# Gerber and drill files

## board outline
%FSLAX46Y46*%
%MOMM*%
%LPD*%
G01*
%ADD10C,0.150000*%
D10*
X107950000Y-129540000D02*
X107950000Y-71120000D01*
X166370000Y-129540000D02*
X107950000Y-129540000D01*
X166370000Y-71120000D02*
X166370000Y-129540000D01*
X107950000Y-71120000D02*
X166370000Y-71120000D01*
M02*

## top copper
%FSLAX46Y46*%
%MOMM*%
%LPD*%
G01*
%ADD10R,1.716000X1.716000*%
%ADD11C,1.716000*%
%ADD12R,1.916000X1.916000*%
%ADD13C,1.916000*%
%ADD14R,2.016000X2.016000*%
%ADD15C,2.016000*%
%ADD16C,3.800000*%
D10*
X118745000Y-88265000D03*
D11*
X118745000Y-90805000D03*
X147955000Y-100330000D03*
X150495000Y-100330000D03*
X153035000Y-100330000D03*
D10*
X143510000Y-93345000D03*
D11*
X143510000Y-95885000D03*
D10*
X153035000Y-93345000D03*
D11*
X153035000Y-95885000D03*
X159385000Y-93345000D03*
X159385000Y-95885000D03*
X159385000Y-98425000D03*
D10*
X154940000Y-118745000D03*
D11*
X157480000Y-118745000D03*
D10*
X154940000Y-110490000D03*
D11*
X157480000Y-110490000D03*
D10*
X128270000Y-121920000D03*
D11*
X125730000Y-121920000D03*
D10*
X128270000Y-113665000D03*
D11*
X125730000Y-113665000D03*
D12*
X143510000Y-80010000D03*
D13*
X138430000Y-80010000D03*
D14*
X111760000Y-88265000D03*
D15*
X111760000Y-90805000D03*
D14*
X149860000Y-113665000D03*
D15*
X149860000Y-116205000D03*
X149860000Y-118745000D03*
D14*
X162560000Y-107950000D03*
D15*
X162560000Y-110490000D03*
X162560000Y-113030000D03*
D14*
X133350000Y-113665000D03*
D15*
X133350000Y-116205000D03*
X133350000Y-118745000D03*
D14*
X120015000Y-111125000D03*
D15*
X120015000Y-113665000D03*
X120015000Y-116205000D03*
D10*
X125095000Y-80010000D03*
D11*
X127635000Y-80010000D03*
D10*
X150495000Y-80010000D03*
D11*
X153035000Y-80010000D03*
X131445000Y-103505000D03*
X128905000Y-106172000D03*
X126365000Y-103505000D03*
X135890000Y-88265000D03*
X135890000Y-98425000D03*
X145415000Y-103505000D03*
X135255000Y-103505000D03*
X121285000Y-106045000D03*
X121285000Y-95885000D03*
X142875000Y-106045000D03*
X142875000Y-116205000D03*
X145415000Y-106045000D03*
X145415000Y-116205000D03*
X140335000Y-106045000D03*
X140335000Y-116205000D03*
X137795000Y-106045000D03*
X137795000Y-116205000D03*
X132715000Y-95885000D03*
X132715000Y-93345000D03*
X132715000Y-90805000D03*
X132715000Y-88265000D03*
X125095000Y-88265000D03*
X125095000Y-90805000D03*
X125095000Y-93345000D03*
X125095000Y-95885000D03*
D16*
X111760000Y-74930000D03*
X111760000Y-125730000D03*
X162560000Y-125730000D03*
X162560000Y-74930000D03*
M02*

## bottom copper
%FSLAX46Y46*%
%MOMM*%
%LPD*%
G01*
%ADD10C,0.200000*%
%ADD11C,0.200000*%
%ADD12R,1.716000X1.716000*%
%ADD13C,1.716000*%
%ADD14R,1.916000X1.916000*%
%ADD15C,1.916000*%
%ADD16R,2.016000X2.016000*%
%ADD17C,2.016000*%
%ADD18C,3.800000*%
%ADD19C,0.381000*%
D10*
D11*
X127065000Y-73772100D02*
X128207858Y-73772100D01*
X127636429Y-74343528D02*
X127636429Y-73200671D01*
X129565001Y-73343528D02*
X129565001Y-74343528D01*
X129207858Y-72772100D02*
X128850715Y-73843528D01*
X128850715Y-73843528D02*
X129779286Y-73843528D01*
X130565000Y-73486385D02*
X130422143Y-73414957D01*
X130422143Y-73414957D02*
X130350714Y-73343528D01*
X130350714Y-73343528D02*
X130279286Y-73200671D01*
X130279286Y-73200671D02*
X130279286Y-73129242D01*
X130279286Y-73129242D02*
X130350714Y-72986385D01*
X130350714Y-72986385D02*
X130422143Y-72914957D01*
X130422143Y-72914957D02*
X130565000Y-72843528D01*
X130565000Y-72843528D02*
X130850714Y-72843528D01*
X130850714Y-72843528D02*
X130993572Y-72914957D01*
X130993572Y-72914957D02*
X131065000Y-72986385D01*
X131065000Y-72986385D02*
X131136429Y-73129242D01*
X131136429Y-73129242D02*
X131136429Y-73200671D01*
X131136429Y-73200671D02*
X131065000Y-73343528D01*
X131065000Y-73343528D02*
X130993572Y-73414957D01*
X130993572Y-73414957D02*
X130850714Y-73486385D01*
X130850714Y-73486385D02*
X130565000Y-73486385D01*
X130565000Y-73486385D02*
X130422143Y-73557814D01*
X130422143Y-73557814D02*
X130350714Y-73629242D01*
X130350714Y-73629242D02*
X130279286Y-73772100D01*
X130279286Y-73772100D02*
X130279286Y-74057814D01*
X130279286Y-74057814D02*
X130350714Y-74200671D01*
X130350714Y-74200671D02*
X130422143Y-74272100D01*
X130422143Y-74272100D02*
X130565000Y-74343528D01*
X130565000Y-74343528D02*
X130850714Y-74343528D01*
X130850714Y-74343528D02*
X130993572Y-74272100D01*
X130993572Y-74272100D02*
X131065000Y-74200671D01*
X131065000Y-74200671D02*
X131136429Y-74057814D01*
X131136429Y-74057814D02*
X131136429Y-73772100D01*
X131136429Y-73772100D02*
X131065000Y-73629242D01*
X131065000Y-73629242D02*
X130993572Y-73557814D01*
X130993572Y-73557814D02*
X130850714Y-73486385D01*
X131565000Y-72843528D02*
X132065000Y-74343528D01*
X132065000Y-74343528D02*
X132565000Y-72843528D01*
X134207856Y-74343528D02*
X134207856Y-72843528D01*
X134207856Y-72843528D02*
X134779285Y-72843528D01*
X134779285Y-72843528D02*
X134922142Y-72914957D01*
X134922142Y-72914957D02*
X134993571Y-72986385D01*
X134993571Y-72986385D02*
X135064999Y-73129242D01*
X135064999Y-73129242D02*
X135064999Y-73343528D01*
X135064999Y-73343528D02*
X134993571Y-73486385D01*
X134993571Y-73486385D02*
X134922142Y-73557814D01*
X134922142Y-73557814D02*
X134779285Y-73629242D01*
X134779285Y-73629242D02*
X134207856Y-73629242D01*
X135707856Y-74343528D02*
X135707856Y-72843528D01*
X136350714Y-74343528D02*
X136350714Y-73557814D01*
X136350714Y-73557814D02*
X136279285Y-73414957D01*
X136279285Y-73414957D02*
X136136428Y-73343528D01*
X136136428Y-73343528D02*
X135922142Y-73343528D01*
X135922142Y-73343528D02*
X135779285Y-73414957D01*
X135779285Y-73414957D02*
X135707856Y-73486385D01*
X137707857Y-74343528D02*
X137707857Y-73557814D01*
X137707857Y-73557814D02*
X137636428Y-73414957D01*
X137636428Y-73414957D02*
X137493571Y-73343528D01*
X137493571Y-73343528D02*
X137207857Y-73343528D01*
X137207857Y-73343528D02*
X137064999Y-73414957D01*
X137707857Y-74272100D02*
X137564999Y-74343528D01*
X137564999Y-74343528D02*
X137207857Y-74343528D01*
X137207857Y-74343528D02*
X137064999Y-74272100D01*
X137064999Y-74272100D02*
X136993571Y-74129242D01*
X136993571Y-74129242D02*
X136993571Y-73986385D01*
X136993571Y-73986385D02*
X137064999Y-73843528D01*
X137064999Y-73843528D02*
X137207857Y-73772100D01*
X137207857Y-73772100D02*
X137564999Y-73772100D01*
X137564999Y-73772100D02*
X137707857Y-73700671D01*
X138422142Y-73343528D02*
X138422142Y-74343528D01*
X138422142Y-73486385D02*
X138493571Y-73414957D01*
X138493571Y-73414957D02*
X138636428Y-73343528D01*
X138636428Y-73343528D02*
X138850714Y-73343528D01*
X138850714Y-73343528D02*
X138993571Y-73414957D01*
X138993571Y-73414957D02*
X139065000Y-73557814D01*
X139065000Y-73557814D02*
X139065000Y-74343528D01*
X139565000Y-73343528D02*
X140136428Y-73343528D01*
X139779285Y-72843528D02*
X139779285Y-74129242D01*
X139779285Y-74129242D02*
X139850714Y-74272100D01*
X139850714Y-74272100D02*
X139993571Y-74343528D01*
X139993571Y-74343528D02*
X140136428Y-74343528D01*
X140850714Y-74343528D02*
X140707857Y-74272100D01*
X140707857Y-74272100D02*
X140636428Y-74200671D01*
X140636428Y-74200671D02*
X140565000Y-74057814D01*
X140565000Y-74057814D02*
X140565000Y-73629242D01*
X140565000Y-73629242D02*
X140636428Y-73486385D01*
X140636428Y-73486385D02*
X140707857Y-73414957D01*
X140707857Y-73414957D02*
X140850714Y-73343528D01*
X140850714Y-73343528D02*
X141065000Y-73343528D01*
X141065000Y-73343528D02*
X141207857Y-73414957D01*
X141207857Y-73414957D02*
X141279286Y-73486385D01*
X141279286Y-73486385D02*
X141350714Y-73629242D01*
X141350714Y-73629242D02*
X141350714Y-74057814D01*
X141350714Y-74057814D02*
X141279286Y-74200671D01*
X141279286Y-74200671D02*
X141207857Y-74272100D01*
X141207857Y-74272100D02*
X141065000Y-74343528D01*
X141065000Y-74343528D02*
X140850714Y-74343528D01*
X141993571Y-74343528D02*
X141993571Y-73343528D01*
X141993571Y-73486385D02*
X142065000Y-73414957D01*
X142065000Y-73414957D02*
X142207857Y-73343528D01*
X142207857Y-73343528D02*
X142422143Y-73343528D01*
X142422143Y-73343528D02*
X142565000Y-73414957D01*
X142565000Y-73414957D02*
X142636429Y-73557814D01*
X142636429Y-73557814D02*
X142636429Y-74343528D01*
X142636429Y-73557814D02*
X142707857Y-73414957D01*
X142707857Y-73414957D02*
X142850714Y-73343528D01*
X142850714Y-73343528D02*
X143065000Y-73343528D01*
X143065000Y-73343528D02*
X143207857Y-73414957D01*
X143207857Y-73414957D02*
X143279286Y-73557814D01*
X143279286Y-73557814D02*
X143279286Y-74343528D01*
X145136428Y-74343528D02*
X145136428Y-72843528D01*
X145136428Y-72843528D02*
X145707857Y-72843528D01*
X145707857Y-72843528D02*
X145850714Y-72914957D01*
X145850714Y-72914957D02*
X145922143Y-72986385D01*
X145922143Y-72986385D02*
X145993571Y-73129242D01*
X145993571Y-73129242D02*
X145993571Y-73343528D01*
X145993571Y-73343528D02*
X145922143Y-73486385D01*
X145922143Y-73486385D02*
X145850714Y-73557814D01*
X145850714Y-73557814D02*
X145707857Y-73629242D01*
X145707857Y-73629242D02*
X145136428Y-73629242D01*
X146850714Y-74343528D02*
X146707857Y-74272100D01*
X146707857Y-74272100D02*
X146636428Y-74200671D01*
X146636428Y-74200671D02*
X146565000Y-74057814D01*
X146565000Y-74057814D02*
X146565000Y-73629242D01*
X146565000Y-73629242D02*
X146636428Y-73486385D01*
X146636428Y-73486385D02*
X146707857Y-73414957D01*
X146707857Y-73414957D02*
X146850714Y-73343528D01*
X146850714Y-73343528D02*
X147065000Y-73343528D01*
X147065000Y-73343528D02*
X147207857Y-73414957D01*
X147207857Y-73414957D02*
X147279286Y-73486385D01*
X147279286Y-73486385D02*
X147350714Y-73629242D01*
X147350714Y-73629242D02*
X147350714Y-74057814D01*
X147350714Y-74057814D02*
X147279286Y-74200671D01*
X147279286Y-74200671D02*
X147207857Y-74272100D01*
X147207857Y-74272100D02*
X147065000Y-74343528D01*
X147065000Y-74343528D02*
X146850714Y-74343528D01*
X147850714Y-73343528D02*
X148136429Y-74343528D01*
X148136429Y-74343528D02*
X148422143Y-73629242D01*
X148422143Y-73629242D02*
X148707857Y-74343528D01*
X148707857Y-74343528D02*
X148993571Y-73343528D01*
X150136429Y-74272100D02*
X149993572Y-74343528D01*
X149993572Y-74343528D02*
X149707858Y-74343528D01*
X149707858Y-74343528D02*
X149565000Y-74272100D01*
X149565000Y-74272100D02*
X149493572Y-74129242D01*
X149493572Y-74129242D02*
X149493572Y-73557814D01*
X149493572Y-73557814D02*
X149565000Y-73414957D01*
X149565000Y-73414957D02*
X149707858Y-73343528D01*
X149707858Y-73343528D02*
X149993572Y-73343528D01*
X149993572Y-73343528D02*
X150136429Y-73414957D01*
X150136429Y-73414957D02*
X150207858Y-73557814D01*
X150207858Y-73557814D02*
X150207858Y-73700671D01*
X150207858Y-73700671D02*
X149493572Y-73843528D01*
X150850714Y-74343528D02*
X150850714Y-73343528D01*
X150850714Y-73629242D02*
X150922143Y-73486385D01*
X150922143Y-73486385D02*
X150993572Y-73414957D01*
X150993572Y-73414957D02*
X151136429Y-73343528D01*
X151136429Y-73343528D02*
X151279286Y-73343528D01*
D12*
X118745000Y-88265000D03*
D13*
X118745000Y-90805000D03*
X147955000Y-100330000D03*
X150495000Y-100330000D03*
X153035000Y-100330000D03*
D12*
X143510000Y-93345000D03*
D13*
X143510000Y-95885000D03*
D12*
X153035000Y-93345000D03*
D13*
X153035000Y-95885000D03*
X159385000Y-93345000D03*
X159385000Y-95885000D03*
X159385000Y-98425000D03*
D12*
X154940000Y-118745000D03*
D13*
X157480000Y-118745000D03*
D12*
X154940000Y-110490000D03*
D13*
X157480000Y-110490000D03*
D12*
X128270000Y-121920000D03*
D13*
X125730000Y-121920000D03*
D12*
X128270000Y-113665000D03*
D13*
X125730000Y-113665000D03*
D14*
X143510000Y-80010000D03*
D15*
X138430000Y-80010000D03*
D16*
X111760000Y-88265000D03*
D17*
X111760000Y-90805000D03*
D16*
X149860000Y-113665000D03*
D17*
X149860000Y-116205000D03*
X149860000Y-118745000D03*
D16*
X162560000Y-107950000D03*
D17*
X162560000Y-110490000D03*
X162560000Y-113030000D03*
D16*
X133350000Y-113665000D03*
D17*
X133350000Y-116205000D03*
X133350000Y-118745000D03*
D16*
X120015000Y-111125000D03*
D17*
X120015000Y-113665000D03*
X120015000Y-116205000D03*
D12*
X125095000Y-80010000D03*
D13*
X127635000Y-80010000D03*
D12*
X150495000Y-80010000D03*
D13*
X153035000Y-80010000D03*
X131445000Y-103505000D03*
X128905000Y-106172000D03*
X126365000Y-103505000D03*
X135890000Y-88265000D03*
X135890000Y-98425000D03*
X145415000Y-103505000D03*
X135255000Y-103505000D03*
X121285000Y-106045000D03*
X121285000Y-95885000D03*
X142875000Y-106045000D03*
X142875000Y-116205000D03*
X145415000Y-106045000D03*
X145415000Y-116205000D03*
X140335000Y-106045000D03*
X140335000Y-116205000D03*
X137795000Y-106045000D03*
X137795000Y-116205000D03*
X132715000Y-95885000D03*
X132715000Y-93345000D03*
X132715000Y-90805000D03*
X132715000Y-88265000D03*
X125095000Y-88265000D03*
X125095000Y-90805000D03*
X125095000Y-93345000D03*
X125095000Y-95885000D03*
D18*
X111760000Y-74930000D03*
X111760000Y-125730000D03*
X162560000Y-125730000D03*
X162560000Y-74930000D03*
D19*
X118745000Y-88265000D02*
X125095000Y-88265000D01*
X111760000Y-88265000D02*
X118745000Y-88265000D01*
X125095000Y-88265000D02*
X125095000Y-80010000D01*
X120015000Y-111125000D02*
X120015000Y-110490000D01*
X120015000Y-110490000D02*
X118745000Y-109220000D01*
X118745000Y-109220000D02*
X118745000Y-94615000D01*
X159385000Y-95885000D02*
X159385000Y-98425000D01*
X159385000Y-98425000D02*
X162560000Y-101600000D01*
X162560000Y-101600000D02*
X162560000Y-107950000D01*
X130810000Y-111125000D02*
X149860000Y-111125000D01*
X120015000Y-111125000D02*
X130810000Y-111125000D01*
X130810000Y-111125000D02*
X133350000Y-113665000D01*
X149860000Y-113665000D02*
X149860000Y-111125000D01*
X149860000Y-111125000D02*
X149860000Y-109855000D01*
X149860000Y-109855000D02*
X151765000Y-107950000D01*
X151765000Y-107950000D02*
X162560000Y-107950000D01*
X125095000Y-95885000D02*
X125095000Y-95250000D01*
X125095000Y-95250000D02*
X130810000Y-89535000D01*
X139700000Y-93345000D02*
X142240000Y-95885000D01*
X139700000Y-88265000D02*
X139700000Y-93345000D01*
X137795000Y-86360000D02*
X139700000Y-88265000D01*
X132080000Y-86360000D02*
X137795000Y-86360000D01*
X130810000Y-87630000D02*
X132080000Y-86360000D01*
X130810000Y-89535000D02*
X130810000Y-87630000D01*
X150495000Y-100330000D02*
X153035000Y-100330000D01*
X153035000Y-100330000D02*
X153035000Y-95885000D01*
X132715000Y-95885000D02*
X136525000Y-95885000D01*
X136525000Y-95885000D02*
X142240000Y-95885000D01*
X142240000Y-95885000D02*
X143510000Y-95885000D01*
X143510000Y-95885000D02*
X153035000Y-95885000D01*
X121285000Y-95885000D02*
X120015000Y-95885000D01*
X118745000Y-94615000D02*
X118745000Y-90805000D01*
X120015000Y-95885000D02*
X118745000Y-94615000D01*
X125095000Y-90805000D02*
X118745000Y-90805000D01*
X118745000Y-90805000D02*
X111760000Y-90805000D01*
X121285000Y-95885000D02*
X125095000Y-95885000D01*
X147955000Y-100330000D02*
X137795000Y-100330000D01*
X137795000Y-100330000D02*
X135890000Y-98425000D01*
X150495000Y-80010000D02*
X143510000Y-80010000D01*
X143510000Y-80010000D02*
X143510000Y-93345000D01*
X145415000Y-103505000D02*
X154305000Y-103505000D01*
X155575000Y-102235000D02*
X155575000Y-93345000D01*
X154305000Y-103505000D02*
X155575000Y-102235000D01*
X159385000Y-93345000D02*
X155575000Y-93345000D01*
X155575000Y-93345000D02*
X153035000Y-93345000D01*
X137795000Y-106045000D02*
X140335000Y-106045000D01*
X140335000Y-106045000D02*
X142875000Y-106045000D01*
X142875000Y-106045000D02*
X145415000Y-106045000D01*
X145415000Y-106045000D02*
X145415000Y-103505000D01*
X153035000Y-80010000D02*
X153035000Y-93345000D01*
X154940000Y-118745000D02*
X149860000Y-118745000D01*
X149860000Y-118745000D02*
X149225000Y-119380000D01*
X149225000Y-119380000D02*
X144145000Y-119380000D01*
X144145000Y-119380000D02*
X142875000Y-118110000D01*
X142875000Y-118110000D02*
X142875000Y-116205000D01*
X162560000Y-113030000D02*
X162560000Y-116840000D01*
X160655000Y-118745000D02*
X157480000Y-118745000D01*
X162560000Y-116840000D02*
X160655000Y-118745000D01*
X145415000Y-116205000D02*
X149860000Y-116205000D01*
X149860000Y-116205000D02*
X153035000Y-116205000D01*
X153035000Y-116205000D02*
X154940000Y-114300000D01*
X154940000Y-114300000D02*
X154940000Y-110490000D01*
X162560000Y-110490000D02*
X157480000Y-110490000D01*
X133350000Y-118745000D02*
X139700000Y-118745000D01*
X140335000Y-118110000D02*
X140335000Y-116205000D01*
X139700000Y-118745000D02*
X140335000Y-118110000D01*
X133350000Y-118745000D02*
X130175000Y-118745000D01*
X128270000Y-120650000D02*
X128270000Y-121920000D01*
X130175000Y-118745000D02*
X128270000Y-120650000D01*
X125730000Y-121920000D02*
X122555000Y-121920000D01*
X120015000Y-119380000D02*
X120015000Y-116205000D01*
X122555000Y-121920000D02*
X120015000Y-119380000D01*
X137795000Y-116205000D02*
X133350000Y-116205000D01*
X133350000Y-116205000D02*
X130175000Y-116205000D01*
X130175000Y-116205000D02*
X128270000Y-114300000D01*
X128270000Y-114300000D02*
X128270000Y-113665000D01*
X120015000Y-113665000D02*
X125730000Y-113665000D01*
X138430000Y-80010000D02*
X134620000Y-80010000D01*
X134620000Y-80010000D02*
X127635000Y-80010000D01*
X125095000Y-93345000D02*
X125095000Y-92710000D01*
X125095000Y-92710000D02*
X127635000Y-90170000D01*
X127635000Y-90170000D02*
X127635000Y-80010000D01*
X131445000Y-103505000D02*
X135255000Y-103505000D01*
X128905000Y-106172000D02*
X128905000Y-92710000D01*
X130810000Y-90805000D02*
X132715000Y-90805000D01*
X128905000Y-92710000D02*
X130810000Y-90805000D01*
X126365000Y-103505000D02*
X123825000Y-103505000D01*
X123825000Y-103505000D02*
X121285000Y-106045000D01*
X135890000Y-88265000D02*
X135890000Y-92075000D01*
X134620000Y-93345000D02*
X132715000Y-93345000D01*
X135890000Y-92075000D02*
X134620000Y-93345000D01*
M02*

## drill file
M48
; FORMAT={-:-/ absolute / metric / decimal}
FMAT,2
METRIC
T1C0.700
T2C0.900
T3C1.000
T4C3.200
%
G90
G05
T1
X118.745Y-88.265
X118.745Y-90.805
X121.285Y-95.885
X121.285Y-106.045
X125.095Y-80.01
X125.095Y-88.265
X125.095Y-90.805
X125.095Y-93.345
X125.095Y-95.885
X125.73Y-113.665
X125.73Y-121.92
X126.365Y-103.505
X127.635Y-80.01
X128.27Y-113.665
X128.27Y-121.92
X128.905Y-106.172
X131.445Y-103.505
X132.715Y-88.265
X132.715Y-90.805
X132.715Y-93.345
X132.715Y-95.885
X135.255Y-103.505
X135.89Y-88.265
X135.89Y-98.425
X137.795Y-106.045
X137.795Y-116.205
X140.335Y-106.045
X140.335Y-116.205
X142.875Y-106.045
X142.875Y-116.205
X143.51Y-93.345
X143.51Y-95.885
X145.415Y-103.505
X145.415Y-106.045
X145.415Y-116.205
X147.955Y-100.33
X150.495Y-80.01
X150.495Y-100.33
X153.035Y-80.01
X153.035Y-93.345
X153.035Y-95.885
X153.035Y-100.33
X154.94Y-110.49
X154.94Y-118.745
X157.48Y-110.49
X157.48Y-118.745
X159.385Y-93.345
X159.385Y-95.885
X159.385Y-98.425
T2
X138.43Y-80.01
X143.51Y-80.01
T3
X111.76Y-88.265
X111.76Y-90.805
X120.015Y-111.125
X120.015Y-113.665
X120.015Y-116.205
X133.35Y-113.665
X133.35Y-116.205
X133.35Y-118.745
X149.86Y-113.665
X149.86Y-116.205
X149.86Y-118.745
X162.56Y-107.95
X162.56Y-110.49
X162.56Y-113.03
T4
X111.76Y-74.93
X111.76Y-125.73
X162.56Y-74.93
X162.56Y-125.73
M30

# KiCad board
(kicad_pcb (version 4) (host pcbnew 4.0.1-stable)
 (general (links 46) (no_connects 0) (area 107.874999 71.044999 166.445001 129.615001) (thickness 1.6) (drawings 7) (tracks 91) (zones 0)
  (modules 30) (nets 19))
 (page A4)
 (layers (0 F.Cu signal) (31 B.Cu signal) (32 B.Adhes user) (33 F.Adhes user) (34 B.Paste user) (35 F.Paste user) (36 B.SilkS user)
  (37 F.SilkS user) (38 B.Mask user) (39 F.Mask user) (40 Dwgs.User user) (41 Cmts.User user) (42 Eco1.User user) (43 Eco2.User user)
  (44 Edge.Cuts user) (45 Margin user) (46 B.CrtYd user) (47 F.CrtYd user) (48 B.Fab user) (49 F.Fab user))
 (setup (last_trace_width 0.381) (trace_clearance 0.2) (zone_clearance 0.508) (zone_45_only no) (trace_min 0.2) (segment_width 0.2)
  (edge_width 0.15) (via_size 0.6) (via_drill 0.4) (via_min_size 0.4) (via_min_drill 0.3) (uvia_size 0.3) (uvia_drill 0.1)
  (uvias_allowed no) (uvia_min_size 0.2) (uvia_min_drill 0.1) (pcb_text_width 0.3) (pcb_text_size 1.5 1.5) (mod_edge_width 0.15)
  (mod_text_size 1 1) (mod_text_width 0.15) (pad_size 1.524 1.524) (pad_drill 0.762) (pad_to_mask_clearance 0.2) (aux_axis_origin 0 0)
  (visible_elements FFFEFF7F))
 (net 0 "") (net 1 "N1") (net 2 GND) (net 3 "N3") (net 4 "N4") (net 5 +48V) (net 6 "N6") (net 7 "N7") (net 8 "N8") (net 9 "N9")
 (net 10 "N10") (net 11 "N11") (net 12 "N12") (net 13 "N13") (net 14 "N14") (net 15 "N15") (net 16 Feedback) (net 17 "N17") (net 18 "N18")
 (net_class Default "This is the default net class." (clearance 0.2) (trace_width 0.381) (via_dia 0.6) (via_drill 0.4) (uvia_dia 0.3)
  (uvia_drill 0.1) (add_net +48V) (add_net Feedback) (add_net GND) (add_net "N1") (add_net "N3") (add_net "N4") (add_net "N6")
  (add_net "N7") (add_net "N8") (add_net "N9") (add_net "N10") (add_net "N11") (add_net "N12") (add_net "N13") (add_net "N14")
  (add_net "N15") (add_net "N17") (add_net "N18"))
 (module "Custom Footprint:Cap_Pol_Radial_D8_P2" (layer F.Cu) (at 118.745 88.265 270)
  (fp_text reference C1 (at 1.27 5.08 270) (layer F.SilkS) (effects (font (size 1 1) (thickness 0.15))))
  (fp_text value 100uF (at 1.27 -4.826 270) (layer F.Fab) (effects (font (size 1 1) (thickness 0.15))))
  (pad 1 thru_hole rect (at 0 0 270) (size 1.716 1.716) (drill 0.7) (layers *.Cu *.Mask F.SilkS) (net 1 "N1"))
  (pad 2 thru_hole circle (at 2.54 0 270) (size 1.716 1.716) (drill 0.7) (layers *.Cu *.Mask F.SilkS) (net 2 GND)))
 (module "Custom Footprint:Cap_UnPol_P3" (layer F.Cu) (at 147.955 100.33 90)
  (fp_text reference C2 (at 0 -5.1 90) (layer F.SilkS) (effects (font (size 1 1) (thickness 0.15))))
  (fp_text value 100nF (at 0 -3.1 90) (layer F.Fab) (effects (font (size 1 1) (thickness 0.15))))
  (pad 1 thru_hole circle (at 0 0 90) (size 1.716 1.716) (drill 0.7) (layers *.Cu *.Mask F.SilkS) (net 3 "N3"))
  (pad 2 thru_hole circle (at 0 2.54 90) (size 1.716 1.716) (drill 0.7) (layers *.Cu *.Mask F.SilkS) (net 2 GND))
  (pad 2 thru_hole circle (at 0 5.08 90) (size 1.716 1.716) (drill 0.7) (layers *.Cu *.Mask F.SilkS) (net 2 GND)))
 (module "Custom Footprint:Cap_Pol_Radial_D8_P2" (layer F.Cu) (at 143.51 93.345 270)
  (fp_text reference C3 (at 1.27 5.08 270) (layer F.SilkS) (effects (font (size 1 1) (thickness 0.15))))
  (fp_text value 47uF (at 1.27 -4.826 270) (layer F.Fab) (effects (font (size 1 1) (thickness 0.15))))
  (pad 1 thru_hole rect (at 0 0 270) (size 1.716 1.716) (drill 0.7) (layers *.Cu *.Mask F.SilkS) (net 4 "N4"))
  (pad 2 thru_hole circle (at 2.54 0 270) (size 1.716 1.716) (drill 0.7) (layers *.Cu *.Mask F.SilkS) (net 2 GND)))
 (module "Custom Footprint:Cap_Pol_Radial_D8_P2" (layer F.Cu) (at 153.035 93.345 270)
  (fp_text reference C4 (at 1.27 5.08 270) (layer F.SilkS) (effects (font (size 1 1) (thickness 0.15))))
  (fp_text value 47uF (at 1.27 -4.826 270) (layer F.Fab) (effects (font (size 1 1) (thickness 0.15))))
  (pad 1 thru_hole rect (at 0 0 270) (size 1.716 1.716) (drill 0.7) (layers *.Cu *.Mask F.SilkS) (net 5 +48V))
  (pad 2 thru_hole circle (at 2.54 0 270) (size 1.716 1.716) (drill 0.7) (layers *.Cu *.Mask F.SilkS) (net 2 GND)))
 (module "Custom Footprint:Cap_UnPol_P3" (layer F.Cu) (at 159.385 93.345)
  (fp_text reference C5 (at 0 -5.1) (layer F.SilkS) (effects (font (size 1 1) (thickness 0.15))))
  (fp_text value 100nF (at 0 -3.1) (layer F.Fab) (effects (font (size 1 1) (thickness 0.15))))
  (pad 1 thru_hole circle (at 0 0) (size 1.716 1.716) (drill 0.7) (layers *.Cu *.Mask F.SilkS) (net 5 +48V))
  (pad 2 thru_hole circle (at 0 2.54) (size 1.716 1.716) (drill 0.7) (layers *.Cu *.Mask F.SilkS) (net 2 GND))
  (pad 2 thru_hole circle (at 0 5.08) (size 1.716 1.716) (drill 0.7) (layers *.Cu *.Mask F.SilkS) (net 2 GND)))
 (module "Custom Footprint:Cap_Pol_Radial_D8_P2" (layer F.Cu) (at 154.94 118.745)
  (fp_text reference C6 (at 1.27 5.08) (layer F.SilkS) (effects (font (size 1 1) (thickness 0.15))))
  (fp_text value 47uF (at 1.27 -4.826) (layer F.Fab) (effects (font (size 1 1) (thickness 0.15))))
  (pad 1 thru_hole rect (at 0 0) (size 1.716 1.716) (drill 0.7) (layers *.Cu *.Mask F.SilkS) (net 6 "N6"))
  (pad 2 thru_hole circle (at 2.54 0) (size 1.716 1.716) (drill 0.7) (layers *.Cu *.Mask F.SilkS) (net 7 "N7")))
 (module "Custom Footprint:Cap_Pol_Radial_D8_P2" (layer F.Cu) (at 154.94 110.49)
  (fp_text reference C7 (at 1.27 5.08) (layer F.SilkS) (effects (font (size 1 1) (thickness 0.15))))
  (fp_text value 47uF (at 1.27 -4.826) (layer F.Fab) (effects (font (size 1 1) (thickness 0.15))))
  (pad 1 thru_hole rect (at 0 0) (size 1.716 1.716) (drill 0.7) (layers *.Cu *.Mask F.SilkS) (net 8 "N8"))
  (pad 2 thru_hole circle (at 2.54 0) (size 1.716 1.716) (drill 0.7) (layers *.Cu *.Mask F.SilkS) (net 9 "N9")))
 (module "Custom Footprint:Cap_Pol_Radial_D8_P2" (layer F.Cu) (at 128.27 121.92 180)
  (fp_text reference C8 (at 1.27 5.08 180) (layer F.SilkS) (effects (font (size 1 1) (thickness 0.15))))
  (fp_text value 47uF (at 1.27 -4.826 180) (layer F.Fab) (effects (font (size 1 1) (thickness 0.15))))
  (pad 1 thru_hole rect (at 0 0 180) (size 1.716 1.716) (drill 0.7) (layers *.Cu *.Mask F.SilkS) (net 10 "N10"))
  (pad 2 thru_hole circle (at 2.54 0 180) (size 1.716 1.716) (drill 0.7) (layers *.Cu *.Mask F.SilkS) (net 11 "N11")))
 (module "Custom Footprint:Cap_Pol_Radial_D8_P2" (layer F.Cu) (at 128.27 113.665 180)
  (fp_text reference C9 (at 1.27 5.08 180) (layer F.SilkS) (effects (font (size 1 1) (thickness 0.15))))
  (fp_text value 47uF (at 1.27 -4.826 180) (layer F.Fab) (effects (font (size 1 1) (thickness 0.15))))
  (pad 1 thru_hole rect (at 0 0 180) (size 1.716 1.716) (drill 0.7) (layers *.Cu *.Mask F.SilkS) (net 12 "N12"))
  (pad 2 thru_hole circle (at 2.54 0 180) (size 1.716 1.716) (drill 0.7) (layers *.Cu *.Mask F.SilkS) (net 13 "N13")))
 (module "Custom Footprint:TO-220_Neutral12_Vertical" (layer F.Cu) (at 140.97 80.01 180)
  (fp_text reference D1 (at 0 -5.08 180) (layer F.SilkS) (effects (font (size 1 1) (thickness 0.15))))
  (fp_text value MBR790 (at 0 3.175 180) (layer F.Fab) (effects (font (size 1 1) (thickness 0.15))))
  (pad 1 thru_hole rect (at -2.54 0 270) (size 1.916 1.916) (drill 0.9) (layers *.Cu *.Mask F.SilkS) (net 4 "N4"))
  (pad 2 thru_hole circle (at 2.54 0 270) (size 1.916 1.916) (drill 0.9) (layers *.Cu *.Mask F.SilkS) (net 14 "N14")))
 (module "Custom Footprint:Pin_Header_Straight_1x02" (layer F.Cu) (at 111.76 88.265)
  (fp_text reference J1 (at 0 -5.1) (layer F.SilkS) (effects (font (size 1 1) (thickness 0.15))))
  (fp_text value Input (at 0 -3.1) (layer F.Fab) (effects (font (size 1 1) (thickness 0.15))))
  (pad 1 thru_hole rect (at 0 0) (size 2.016 2.016) (drill 1) (layers *.Cu *.Mask F.SilkS) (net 1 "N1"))
  (pad 2 thru_hole circle (at 0 2.54) (size 2.016 2.016) (drill 1) (layers *.Cu *.Mask F.SilkS) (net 2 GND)))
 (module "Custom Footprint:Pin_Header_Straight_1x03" (layer F.Cu) (at 149.86 113.665)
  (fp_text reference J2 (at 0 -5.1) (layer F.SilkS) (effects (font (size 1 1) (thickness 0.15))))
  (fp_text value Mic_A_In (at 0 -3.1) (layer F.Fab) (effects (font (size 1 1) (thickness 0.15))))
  (pad 1 thru_hole rect (at 0 0) (size 2.016 2.016) (drill 1) (layers *.Cu *.Mask F.SilkS) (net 2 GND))
  (pad 2 thru_hole circle (at 0 2.54) (size 2.016 2.016) (drill 1) (layers *.Cu *.Mask F.SilkS) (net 8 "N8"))
  (pad 3 thru_hole circle (at 0 5.08) (size 2.016 2.016) (drill 1) (layers *.Cu *.Mask F.SilkS) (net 6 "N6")))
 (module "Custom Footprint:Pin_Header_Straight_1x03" (layer F.Cu) (at 162.56 107.95)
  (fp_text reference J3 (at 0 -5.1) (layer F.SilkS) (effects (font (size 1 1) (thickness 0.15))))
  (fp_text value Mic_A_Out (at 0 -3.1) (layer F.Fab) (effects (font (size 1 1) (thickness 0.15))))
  (pad 1 thru_hole rect (at 0 0) (size 2.016 2.016) (drill 1) (layers *.Cu *.Mask F.SilkS) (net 2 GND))
  (pad 2 thru_hole circle (at 0 2.54) (size 2.016 2.016) (drill 1) (layers *.Cu *.Mask F.SilkS) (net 9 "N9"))
  (pad 3 thru_hole circle (at 0 5.08) (size 2.016 2.016) (drill 1) (layers *.Cu *.Mask F.SilkS) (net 7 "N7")))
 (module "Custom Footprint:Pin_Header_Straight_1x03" (layer F.Cu) (at 133.35 113.665)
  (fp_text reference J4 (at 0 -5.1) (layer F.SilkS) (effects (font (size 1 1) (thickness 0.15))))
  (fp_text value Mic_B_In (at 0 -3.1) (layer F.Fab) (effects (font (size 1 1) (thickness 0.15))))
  (pad 1 thru_hole rect (at 0 0) (size 2.016 2.016) (drill 1) (layers *.Cu *.Mask F.SilkS) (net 2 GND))
  (pad 2 thru_hole circle (at 0 2.54) (size 2.016 2.016) (drill 1) (layers *.Cu *.Mask F.SilkS) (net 12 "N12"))
  (pad 3 thru_hole circle (at 0 5.08) (size 2.016 2.016) (drill 1) (layers *.Cu *.Mask F.SilkS) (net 10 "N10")))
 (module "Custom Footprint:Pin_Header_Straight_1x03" (layer F.Cu) (at 120.015 111.125)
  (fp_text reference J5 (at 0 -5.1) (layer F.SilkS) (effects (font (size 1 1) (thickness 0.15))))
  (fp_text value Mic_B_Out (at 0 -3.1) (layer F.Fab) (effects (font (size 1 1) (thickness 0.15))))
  (pad 1 thru_hole rect (at 0 0) (size 2.016 2.016) (drill 1) (layers *.Cu *.Mask F.SilkS) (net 2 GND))
  (pad 2 thru_hole circle (at 0 2.54) (size 2.016 2.016) (drill 1) (layers *.Cu *.Mask F.SilkS) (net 13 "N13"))
  (pad 3 thru_hole circle (at 0 5.08) (size 2.016 2.016) (drill 1) (layers *.Cu *.Mask F.SilkS) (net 11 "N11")))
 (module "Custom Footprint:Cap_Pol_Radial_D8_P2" (layer F.Cu) (at 125.095 80.01)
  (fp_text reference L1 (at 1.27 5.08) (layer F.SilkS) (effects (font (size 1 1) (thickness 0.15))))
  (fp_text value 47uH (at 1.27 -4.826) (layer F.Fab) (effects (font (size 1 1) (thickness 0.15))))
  (pad 1 thru_hole rect (at 0 0) (size 1.716 1.716) (drill 0.7) (layers *.Cu *.Mask F.SilkS) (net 1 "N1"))
  (pad 2 thru_hole circle (at 2.54 0) (size 1.716 1.716) (drill 0.7) (layers *.Cu *.Mask F.SilkS) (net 14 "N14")))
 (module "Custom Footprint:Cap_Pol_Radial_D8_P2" (layer F.Cu) (at 150.495 80.01)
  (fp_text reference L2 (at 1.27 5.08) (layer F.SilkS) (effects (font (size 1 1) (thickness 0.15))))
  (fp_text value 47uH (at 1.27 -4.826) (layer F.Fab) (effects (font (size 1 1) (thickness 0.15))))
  (pad 1 thru_hole rect (at 0 0) (size 1.716 1.716) (drill 0.7) (layers *.Cu *.Mask F.SilkS) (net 4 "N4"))
  (pad 2 thru_hole circle (at 2.54 0) (size 1.716 1.716) (drill 0.7) (layers *.Cu *.Mask F.SilkS) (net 5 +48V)))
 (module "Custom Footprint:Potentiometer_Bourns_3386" (layer F.Cu) (at 131.445 103.505)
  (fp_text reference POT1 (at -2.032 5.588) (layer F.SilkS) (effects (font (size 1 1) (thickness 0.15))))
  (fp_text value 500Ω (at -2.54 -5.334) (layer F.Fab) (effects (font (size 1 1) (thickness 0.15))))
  (pad 1 thru_hole circle (at 0 0) (size 1.716 1.716) (drill 0.7) (layers *.Cu *.Mask F.SilkS) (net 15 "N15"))
  (pad 2 thru_hole circle (at -2.54 2.667) (size 1.716 1.716) (drill 0.7) (layers *.Cu *.Mask F.SilkS) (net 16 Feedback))
  (pad 3 thru_hole circle (at -5.08 0) (size 1.716 1.716) (drill 0.7) (layers *.Cu *.Mask F.SilkS) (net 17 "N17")))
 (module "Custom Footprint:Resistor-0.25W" (layer F.Cu) (at 135.89 88.265 270)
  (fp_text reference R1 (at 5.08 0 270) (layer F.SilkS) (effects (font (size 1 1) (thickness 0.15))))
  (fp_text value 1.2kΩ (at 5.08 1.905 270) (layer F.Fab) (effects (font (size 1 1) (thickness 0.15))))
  (pad 1 thru_hole circle (at 0 0 270) (size 1.716 1.716) (drill 0.7) (layers *.Cu *.Mask F.SilkS) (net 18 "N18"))
  (pad 2 thru_hole circle (at 10.16 0 270) (size 1.716 1.716) (drill 0.7) (layers *.Cu *.Mask F.SilkS) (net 3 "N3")))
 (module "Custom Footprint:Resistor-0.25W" (layer F.Cu) (at 145.415 103.505 180)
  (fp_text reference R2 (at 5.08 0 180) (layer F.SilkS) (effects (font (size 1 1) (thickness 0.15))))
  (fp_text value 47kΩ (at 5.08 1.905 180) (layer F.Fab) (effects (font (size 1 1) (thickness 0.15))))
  (pad 1 thru_hole circle (at 0 0 180) (size 1.716 1.716) (drill 0.7) (layers *.Cu *.Mask F.SilkS) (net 5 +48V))
  (pad 2 thru_hole circle (at 10.16 0 180) (size 1.716 1.716) (drill 0.7) (layers *.Cu *.Mask F.SilkS) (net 15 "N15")))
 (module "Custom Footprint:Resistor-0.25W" (layer F.Cu) (at 121.285 106.045 90)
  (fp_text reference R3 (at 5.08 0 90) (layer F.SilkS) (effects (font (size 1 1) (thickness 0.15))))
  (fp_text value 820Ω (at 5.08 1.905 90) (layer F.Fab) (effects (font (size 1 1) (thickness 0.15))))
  (pad 1 thru_hole circle (at 0 0 90) (size 1.716 1.716) (drill 0.7) (layers *.Cu *.Mask F.SilkS) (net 17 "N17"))
  (pad 2 thru_hole circle (at 10.16 0 90) (size 1.716 1.716) (drill 0.7) (layers *.Cu *.Mask F.SilkS) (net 2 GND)))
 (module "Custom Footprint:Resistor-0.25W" (layer F.Cu) (at 142.875 106.045 270)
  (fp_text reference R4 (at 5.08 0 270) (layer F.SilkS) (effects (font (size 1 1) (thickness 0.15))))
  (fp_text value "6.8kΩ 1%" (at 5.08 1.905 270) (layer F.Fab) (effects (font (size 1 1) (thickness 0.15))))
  (pad 1 thru_hole circle (at 0 0 270) (size 1.716 1.716) (drill 0.7) (layers *.Cu *.Mask F.SilkS) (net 5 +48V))
  (pad 2 thru_hole circle (at 10.16 0 270) (size 1.716 1.716) (drill 0.7) (layers *.Cu *.Mask F.SilkS) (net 6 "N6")))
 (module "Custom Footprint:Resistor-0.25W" (layer F.Cu) (at 145.415 106.045 270)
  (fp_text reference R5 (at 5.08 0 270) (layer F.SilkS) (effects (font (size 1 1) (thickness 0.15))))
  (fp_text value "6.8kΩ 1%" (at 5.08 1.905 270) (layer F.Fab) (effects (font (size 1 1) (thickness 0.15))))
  (pad 1 thru_hole circle (at 0 0 270) (size 1.716 1.716) (drill 0.7) (layers *.Cu *.Mask F.SilkS) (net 5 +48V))
  (pad 2 thru_hole circle (at 10.16 0 270) (size 1.716 1.716) (drill 0.7) (layers *.Cu *.Mask F.SilkS) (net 8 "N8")))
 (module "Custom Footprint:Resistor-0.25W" (layer F.Cu) (at 140.335 106.045 270)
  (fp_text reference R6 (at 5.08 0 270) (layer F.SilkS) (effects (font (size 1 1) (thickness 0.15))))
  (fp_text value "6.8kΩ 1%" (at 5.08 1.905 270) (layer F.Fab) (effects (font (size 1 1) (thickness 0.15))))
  (pad 1 thru_hole circle (at 0 0 270) (size 1.716 1.716) (drill 0.7) (layers *.Cu *.Mask F.SilkS) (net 5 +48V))
  (pad 2 thru_hole circle (at 10.16 0 270) (size 1.716 1.716) (drill 0.7) (layers *.Cu *.Mask F.SilkS) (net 10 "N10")))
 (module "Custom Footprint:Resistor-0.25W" (layer F.Cu) (at 137.795 106.045 270)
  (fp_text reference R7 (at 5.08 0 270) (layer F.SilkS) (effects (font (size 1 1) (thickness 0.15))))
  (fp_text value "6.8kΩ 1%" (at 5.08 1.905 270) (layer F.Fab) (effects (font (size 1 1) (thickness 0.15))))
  (pad 1 thru_hole circle (at 0 0 270) (size 1.716 1.716) (drill 0.7) (layers *.Cu *.Mask F.SilkS) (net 5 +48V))
  (pad 2 thru_hole circle (at 10.16 0 270) (size 1.716 1.716) (drill 0.7) (layers *.Cu *.Mask F.SilkS) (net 12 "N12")))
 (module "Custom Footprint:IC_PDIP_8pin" (layer F.Cu) (at 128.905 92.075 90)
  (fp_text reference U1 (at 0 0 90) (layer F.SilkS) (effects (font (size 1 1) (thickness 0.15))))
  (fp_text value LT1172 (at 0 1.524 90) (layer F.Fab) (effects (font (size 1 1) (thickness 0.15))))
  (pad 1 thru_hole circle (at -3.81 3.81 90) (size 1.716 1.716) (drill 0.7) (layers *.Cu *.Mask F.SilkS) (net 2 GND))
  (pad 2 thru_hole circle (at -1.27 3.81 90) (size 1.716 1.716) (drill 0.7) (layers *.Cu *.Mask F.SilkS) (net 18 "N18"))
  (pad 3 thru_hole circle (at 1.27 3.81 90) (size 1.716 1.716) (drill 0.7) (layers *.Cu *.Mask F.SilkS) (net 16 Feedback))
  (pad 4 thru_hole circle (at 3.81 3.81 90) (size 1.716 1.716) (drill 0.7) (layers *.Cu *.Mask F.SilkS))
  (pad 5 thru_hole circle (at 3.81 -3.81 90) (size 1.716 1.716) (drill 0.7) (layers *.Cu *.Mask F.SilkS) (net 1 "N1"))
  (pad 6 thru_hole circle (at 1.27 -3.81 90) (size 1.716 1.716) (drill 0.7) (layers *.Cu *.Mask F.SilkS) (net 2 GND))
  (pad 7 thru_hole circle (at -1.27 -3.81 90) (size 1.716 1.716) (drill 0.7) (layers *.Cu *.Mask F.SilkS) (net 14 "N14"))
  (pad 8 thru_hole circle (at -3.81 -3.81 90) (size 1.716 1.716) (drill 0.7) (layers *.Cu *.Mask F.SilkS) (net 2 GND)))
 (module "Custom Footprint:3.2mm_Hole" (layer F.Cu) (at 111.76 74.93)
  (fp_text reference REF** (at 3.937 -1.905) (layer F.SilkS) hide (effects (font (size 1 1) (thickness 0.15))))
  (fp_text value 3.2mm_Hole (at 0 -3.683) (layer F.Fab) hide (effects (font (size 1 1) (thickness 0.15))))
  (pad 1 thru_hole circle (at 0 0) (size 3.8 3.8) (drill 3.2) (layers *.Cu *.Mask F.SilkS)))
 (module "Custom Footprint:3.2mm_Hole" (layer F.Cu) (at 111.76 125.73)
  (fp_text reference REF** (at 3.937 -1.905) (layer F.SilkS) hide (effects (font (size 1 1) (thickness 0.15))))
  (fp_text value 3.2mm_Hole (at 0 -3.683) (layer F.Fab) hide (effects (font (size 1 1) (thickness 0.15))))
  (pad 1 thru_hole circle (at 0 0) (size 3.8 3.8) (drill 3.2) (layers *.Cu *.Mask F.SilkS)))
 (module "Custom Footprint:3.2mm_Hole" (layer F.Cu) (at 162.56 125.73)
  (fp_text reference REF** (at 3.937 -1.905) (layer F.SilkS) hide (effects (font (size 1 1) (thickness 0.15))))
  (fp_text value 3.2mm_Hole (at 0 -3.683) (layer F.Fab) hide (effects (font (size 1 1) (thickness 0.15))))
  (pad 1 thru_hole circle (at 0 0) (size 3.8 3.8) (drill 3.2) (layers *.Cu *.Mask F.SilkS)))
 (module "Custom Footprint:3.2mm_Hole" (layer F.Cu) (at 162.56 74.93)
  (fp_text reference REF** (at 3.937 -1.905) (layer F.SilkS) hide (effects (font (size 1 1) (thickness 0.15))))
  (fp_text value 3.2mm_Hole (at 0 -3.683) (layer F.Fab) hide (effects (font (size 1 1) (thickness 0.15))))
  (pad 1 thru_hole circle (at 0 0) (size 3.8 3.8) (drill 3.2) (layers *.Cu *.Mask F.SilkS)))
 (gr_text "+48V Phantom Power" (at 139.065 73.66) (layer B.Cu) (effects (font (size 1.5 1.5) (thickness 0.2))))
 (gr_line (start 107.95 129.54) (end 107.95 71.12) (angle 90) (layer Edge.Cuts) (width 0.15))
 (gr_line (start 166.37 129.54) (end 107.95 129.54) (angle 90) (layer Edge.Cuts) (width 0.15))
 (gr_line (start 166.37 71.12) (end 166.37 129.54) (angle 90) (layer Edge.Cuts) (width 0.15))
 (gr_line (start 107.95 71.12) (end 166.37 71.12) (angle 90) (layer Edge.Cuts) (width 0.15))
 (segment (start 118.745 88.265) (end 125.095 88.265) (width 0.381) (layer B.Cu) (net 1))
 (segment (start 111.76 88.265) (end 118.745 88.265) (width 0.381) (layer B.Cu) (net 1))
 (segment (start 125.095 88.265) (end 125.095 80.01) (width 0.381) (layer B.Cu) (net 1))
 (segment (start 120.015 111.125) (end 120.015 110.49) (width 0.381) (layer B.Cu) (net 2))
 (segment (start 120.015 110.49) (end 118.745 109.22) (width 0.381) (layer B.Cu) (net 2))
 (segment (start 118.745 109.22) (end 118.745 94.615) (width 0.381) (layer B.Cu) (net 2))
 (segment (start 159.385 95.885) (end 159.385 98.425) (width 0.381) (layer B.Cu) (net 2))
 (segment (start 159.385 98.425) (end 162.56 101.6) (width 0.381) (layer B.Cu) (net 2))
 (segment (start 162.56 101.6) (end 162.56 107.95) (width 0.381) (layer B.Cu) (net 2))
 (segment (start 130.81 111.125) (end 149.86 111.125) (width 0.381) (layer B.Cu) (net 2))
 (segment (start 120.015 111.125) (end 130.81 111.125) (width 0.381) (layer B.Cu) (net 2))
 (segment (start 130.81 111.125) (end 133.35 113.665) (width 0.381) (layer B.Cu) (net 2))
 (segment (start 149.86 113.665) (end 149.86 111.125) (width 0.381) (layer B.Cu) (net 2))
 (segment (start 149.86 111.125) (end 149.86 109.855) (width 0.381) (layer B.Cu) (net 2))
 (segment (start 149.86 109.855) (end 151.765 107.95) (width 0.381) (layer B.Cu) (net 2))
 (segment (start 151.765 107.95) (end 162.56 107.95) (width 0.381) (layer B.Cu) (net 2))
 (segment (start 125.095 95.885) (end 125.095 95.25) (width 0.381) (layer B.Cu) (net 2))
 (segment (start 125.095 95.25) (end 130.81 89.535) (width 0.381) (layer B.Cu) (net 2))
 (segment (start 139.7 93.345) (end 142.24 95.885) (width 0.381) (layer B.Cu) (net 2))
 (segment (start 139.7 88.265) (end 139.7 93.345) (width 0.381) (layer B.Cu) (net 2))
 (segment (start 137.795 86.36) (end 139.7 88.265) (width 0.381) (layer B.Cu) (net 2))
 (segment (start 132.08 86.36) (end 137.795 86.36) (width 0.381) (layer B.Cu) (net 2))
 (segment (start 130.81 87.63) (end 132.08 86.36) (width 0.381) (layer B.Cu) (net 2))
 (segment (start 130.81 89.535) (end 130.81 87.63) (width 0.381) (layer B.Cu) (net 2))
 (segment (start 150.495 100.33) (end 153.035 100.33) (width 0.381) (layer B.Cu) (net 2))
 (segment (start 153.035 100.33) (end 153.035 95.885) (width 0.381) (layer B.Cu) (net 2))
 (segment (start 132.715 95.885) (end 136.525 95.885) (width 0.381) (layer B.Cu) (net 2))
 (segment (start 136.525 95.885) (end 142.24 95.885) (width 0.381) (layer B.Cu) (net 2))
 (segment (start 142.24 95.885) (end 143.51 95.885) (width 0.381) (layer B.Cu) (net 2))
 (segment (start 143.51 95.885) (end 153.035 95.885) (width 0.381) (layer B.Cu) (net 2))
 (segment (start 121.285 95.885) (end 120.015 95.885) (width 0.381) (layer B.Cu) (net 2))
 (segment (start 118.745 94.615) (end 118.745 90.805) (width 0.381) (layer B.Cu) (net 2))
 (segment (start 120.015 95.885) (end 118.745 94.615) (width 0.381) (layer B.Cu) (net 2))
 (segment (start 125.095 90.805) (end 118.745 90.805) (width 0.381) (layer B.Cu) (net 2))
 (segment (start 118.745 90.805) (end 111.76 90.805) (width 0.381) (layer B.Cu) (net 2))
 (segment (start 121.285 95.885) (end 125.095 95.885) (width 0.381) (layer B.Cu) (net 2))
 (segment (start 147.955 100.33) (end 137.795 100.33) (width 0.381) (layer B.Cu) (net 3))
 (segment (start 137.795 100.33) (end 135.89 98.425) (width 0.381) (layer B.Cu) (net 3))
 (segment (start 150.495 80.01) (end 143.51 80.01) (width 0.381) (layer B.Cu) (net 4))
 (segment (start 143.51 80.01) (end 143.51 93.345) (width 0.381) (layer B.Cu) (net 4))
 (segment (start 145.415 103.505) (end 154.305 103.505) (width 0.381) (layer B.Cu) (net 5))
 (segment (start 155.575 102.235) (end 155.575 93.345) (width 0.381) (layer B.Cu) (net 5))
 (segment (start 154.305 103.505) (end 155.575 102.235) (width 0.381) (layer B.Cu) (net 5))
 (segment (start 159.385 93.345) (end 155.575 93.345) (width 0.381) (layer B.Cu) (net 5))
 (segment (start 155.575 93.345) (end 153.035 93.345) (width 0.381) (layer B.Cu) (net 5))
 (segment (start 137.795 106.045) (end 140.335 106.045) (width 0.381) (layer B.Cu) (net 5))
 (segment (start 140.335 106.045) (end 142.875 106.045) (width 0.381) (layer B.Cu) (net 5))
 (segment (start 142.875 106.045) (end 145.415 106.045) (width 0.381) (layer B.Cu) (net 5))
 (segment (start 145.415 106.045) (end 145.415 103.505) (width 0.381) (layer B.Cu) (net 5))
 (segment (start 153.035 80.01) (end 153.035 93.345) (width 0.381) (layer B.Cu) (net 5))
 (segment (start 154.94 118.745) (end 149.86 118.745) (width 0.381) (layer B.Cu) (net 6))
 (segment (start 149.86 118.745) (end 149.225 119.38) (width 0.381) (layer B.Cu) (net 6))
 (segment (start 149.225 119.38) (end 144.145 119.38) (width 0.381) (layer B.Cu) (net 6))
 (segment (start 144.145 119.38) (end 142.875 118.11) (width 0.381) (layer B.Cu) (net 6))
 (segment (start 142.875 118.11) (end 142.875 116.205) (width 0.381) (layer B.Cu) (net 6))
 (segment (start 162.56 113.03) (end 162.56 116.84) (width 0.381) (layer B.Cu) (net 7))
 (segment (start 160.655 118.745) (end 157.48 118.745) (width 0.381) (layer B.Cu) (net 7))
 (segment (start 162.56 116.84) (end 160.655 118.745) (width 0.381) (layer B.Cu) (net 7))
 (segment (start 145.415 116.205) (end 149.86 116.205) (width 0.381) (layer B.Cu) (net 8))
 (segment (start 149.86 116.205) (end 153.035 116.205) (width 0.381) (layer B.Cu) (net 8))
 (segment (start 153.035 116.205) (end 154.94 114.3) (width 0.381) (layer B.Cu) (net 8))
 (segment (start 154.94 114.3) (end 154.94 110.49) (width 0.381) (layer B.Cu) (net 8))
 (segment (start 162.56 110.49) (end 157.48 110.49) (width 0.381) (layer B.Cu) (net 9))
 (segment (start 133.35 118.745) (end 139.7 118.745) (width 0.381) (layer B.Cu) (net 10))
 (segment (start 140.335 118.11) (end 140.335 116.205) (width 0.381) (layer B.Cu) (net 10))
 (segment (start 139.7 118.745) (end 140.335 118.11) (width 0.381) (layer B.Cu) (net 10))
 (segment (start 133.35 118.745) (end 130.175 118.745) (width 0.381) (layer B.Cu) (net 10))
 (segment (start 128.27 120.65) (end 128.27 121.92) (width 0.381) (layer B.Cu) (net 10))
 (segment (start 130.175 118.745) (end 128.27 120.65) (width 0.381) (layer B.Cu) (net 10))
 (segment (start 125.73 121.92) (end 122.555 121.92) (width 0.381) (layer B.Cu) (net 11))
 (segment (start 120.015 119.38) (end 120.015 116.205) (width 0.381) (layer B.Cu) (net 11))
 (segment (start 122.555 121.92) (end 120.015 119.38) (width 0.381) (layer B.Cu) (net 11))
 (segment (start 137.795 116.205) (end 133.35 116.205) (width 0.381) (layer B.Cu) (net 12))
 (segment (start 133.35 116.205) (end 130.175 116.205) (width 0.381) (layer B.Cu) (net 12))
 (segment (start 130.175 116.205) (end 128.27 114.3) (width 0.381) (layer B.Cu) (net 12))
 (segment (start 128.27 114.3) (end 128.27 113.665) (width 0.381) (layer B.Cu) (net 12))
 (segment (start 120.015 113.665) (end 125.73 113.665) (width 0.381) (layer B.Cu) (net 13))
 (segment (start 138.43 80.01) (end 134.62 80.01) (width 0.381) (layer B.Cu) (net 14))
 (segment (start 134.62 80.01) (end 127.635 80.01) (width 0.381) (layer B.Cu) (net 14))
 (segment (start 125.095 93.345) (end 125.095 92.71) (width 0.381) (layer B.Cu) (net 14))
 (segment (start 125.095 92.71) (end 127.635 90.17) (width 0.381) (layer B.Cu) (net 14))
 (segment (start 127.635 90.17) (end 127.635 80.01) (width 0.381) (layer B.Cu) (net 14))
 (segment (start 131.445 103.505) (end 135.255 103.505) (width 0.381) (layer B.Cu) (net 15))
 (segment (start 128.905 106.172) (end 128.905 92.71) (width 0.381) (layer B.Cu) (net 16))
 (segment (start 130.81 90.805) (end 132.715 90.805) (width 0.381) (layer B.Cu) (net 16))
 (segment (start 128.905 92.71) (end 130.81 90.805) (width 0.381) (layer B.Cu) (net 16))
 (segment (start 126.365 103.505) (end 123.825 103.505) (width 0.381) (layer B.Cu) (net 17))
 (segment (start 123.825 103.505) (end 121.285 106.045) (width 0.381) (layer B.Cu) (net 17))
 (segment (start 135.89 88.265) (end 135.89 92.075) (width 0.381) (layer B.Cu) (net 18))
 (segment (start 134.62 93.345) (end 132.715 93.345) (width 0.381) (layer B.Cu) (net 18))
 (segment (start 135.89 92.075) (end 134.62 93.345) (width 0.381) (layer B.Cu) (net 18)))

